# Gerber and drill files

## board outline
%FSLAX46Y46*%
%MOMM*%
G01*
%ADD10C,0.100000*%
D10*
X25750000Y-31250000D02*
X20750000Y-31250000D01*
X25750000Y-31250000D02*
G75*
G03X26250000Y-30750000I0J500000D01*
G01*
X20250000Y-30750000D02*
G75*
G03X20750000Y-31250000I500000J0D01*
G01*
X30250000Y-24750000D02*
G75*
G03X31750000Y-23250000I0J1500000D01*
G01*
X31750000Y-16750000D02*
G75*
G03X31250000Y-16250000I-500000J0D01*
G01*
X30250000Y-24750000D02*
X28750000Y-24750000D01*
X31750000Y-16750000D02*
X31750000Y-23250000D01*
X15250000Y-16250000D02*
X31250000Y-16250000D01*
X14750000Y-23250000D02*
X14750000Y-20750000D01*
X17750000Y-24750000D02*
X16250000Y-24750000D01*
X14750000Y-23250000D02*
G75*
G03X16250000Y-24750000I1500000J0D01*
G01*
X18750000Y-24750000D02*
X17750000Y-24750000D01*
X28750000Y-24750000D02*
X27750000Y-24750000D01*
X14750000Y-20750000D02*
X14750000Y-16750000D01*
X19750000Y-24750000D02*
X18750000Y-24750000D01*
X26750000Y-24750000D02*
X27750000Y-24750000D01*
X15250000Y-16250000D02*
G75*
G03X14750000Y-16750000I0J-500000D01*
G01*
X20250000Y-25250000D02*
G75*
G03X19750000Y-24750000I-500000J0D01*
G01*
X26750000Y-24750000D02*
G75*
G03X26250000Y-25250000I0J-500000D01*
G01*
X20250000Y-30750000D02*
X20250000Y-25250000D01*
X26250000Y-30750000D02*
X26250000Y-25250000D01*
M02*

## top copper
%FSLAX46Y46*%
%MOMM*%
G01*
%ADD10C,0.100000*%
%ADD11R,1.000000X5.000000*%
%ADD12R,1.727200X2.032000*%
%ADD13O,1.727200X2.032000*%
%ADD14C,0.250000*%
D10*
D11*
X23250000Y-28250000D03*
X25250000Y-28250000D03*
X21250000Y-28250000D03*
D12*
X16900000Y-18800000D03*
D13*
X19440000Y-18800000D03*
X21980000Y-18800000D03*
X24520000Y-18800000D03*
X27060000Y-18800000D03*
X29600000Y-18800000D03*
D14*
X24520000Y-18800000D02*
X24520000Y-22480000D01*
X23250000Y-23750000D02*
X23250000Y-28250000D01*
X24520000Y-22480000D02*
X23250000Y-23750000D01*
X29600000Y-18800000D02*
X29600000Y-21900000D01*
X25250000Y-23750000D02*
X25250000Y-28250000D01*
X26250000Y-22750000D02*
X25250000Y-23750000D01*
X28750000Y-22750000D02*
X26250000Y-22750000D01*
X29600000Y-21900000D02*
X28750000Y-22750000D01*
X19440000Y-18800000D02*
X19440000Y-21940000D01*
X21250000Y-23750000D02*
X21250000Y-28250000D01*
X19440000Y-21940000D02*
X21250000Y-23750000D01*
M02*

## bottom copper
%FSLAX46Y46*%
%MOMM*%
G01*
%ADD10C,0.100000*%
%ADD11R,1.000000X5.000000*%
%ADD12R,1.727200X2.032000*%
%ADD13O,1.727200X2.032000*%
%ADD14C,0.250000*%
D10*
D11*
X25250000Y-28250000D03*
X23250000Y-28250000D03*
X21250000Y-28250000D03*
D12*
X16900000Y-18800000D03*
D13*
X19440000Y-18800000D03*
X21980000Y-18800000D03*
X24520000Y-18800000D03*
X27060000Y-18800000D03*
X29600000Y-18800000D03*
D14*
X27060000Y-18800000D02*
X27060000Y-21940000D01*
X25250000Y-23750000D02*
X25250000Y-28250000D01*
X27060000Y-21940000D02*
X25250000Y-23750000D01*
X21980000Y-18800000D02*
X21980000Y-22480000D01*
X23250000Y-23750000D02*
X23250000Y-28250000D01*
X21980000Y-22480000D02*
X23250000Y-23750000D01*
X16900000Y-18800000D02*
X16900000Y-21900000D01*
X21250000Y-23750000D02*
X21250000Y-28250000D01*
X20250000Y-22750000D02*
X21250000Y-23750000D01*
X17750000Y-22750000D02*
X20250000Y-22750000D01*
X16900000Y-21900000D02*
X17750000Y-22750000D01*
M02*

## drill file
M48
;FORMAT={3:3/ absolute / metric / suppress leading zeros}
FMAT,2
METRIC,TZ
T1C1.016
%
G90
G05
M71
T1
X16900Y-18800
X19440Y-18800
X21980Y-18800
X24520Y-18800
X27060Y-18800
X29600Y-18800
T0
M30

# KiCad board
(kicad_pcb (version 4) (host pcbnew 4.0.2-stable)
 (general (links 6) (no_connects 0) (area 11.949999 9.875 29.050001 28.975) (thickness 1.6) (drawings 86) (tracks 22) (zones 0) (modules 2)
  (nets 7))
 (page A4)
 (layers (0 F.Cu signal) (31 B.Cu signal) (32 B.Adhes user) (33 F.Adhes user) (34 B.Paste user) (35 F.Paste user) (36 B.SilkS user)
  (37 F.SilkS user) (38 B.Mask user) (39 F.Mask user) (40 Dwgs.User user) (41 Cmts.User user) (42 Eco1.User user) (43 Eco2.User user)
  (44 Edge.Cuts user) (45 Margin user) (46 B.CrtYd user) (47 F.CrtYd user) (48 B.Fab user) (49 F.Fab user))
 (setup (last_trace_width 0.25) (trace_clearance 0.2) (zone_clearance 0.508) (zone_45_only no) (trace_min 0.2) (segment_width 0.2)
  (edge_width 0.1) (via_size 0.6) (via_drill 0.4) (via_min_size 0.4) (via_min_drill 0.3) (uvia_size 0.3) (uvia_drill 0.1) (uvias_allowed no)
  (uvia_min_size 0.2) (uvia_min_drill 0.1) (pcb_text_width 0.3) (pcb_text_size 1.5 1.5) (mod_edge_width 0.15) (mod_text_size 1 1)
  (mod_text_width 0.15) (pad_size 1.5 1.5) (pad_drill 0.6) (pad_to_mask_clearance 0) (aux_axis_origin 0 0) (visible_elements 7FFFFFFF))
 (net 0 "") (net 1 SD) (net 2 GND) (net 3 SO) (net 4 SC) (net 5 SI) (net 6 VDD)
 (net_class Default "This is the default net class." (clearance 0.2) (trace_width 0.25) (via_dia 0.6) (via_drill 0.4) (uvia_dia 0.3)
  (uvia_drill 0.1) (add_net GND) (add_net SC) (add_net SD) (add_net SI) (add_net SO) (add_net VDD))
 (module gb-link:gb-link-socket (layer F.Cu) (at 20.5 24)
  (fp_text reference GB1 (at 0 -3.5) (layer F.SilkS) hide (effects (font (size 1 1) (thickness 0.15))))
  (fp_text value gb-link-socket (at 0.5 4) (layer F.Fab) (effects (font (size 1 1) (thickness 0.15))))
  (pad 4 connect rect (at 0 0) (size 1 5) (layers F.Cu F.Mask) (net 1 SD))
  (pad 6 connect rect (at 2 0) (size 1 5) (layers F.Cu F.Mask) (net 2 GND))
  (pad 2 connect rect (at -2 0) (size 1 5) (layers F.Cu F.Mask) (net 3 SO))
  (pad 5 connect rect (at 2 0) (size 1 5) (layers B.Cu B.Mask) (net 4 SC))
  (pad 3 connect rect (at 0 0) (size 1 5) (layers B.Cu B.Mask) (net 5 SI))
  (pad 1 connect rect (at -2 0) (size 1 5) (layers B.Cu B.Mask) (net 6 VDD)))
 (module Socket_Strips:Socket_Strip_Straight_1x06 (layer F.Cu) (at 14.15 14.55)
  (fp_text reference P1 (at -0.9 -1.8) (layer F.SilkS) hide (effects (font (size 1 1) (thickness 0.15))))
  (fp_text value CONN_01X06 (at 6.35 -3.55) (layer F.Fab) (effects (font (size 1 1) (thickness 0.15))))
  (pad 1 thru_hole rect (at 0 0) (size 1.7272 2.032) (drill 1.016) (layers *.Cu *.Mask F.SilkS) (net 6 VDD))
  (pad 2 thru_hole oval (at 2.54 0) (size 1.7272 2.032) (drill 1.016) (layers *.Cu *.Mask F.SilkS) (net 3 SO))
  (pad 3 thru_hole oval (at 5.08 0) (size 1.7272 2.032) (drill 1.016) (layers *.Cu *.Mask F.SilkS) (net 5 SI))
  (pad 4 thru_hole oval (at 7.62 0) (size 1.7272 2.032) (drill 1.016) (layers *.Cu *.Mask F.SilkS) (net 1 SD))
  (pad 5 thru_hole oval (at 10.16 0) (size 1.7272 2.032) (drill 1.016) (layers *.Cu *.Mask F.SilkS) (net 4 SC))
  (pad 6 thru_hole oval (at 12.7 0) (size 1.7272 2.032) (drill 1.016) (layers *.Cu *.Mask F.SilkS) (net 2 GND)))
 (gr_line (start 23 27) (end 18 27) (angle 90) (layer Edge.Cuts) (width 0.1))
 (gr_arc (start 23 26.5) (end 23.5 26.5) (angle 90) (layer Edge.Cuts) (width 0.1))
 (gr_arc (start 18 26.5) (end 18 27) (angle 90) (layer Edge.Cuts) (width 0.1))
 (gr_arc (start 27.5 19) (end 29 19) (angle 90) (layer Edge.Cuts) (width 0.1))
 (gr_arc (start 28.5 12.5) (end 28.5 12) (angle 90) (layer Edge.Cuts) (width 0.1))
 (gr_line (start 27.5 20.5) (end 26 20.5) (angle 90) (layer Edge.Cuts) (width 0.1))
 (gr_line (start 29 12.5) (end 29 19) (angle 90) (layer Edge.Cuts) (width 0.1))
 (gr_line (start 12.5 12) (end 28.5 12) (angle 90) (layer Edge.Cuts) (width 0.1))
 (gr_line (start 12 19) (end 12 16.5) (angle 90) (layer Edge.Cuts) (width 0.1))
 (gr_line (start 15 20.5) (end 13.5 20.5) (angle 90) (layer Edge.Cuts) (width 0.1))
 (gr_arc (start 13.5 19) (end 13.5 20.5) (angle 90) (layer Edge.Cuts) (width 0.1))
 (gr_line (start 16 20.5) (end 15 20.5) (angle 90) (layer Edge.Cuts) (width 0.1))
 (gr_line (start 26 20.5) (end 25 20.5) (angle 90) (layer Edge.Cuts) (width 0.1))
 (gr_line (start 12 16.5) (end 12 12.5) (angle 90) (layer Edge.Cuts) (width 0.1))
 (gr_line (start 17 20.5) (end 16 20.5) (angle 90) (layer Edge.Cuts) (width 0.1))
 (gr_line (start 24 20.5) (end 25 20.5) (angle 90) (layer Edge.Cuts) (width 0.1))
 (gr_arc (start 12.5 12.5) (end 12 12.5) (angle 90) (layer Edge.Cuts) (width 0.1))
 (gr_arc (start 17 21) (end 17 20.5) (angle 90) (layer Edge.Cuts) (width 0.1))
 (gr_arc (start 24 21) (end 23.5 21) (angle 90) (layer Edge.Cuts) (width 0.1))
 (gr_line (start 17.5 26.5) (end 17.5 21) (angle 90) (layer Edge.Cuts) (width 0.1))
 (gr_line (start 23.5 26.5) (end 23.5 21) (angle 90) (layer Edge.Cuts) (width 0.1))
 (segment (start 21.77 14.55) (end 21.77 18.23) (width 0.25) (layer F.Cu) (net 1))
 (segment (start 20.5 19.5) (end 20.5 24) (width 0.25) (layer F.Cu) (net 1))
 (segment (start 21.77 18.23) (end 20.5 19.5) (width 0.25) (layer F.Cu) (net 1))
 (segment (start 26.85 14.55) (end 26.85 17.65) (width 0.25) (layer F.Cu) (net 2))
 (segment (start 22.5 19.5) (end 22.5 24) (width 0.25) (layer F.Cu) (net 2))
 (segment (start 23.5 18.5) (end 22.5 19.5) (width 0.25) (layer F.Cu) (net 2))
 (segment (start 26 18.5) (end 23.5 18.5) (width 0.25) (layer F.Cu) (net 2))
 (segment (start 26.85 17.65) (end 26 18.5) (width 0.25) (layer F.Cu) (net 2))
 (segment (start 16.69 14.55) (end 16.69 17.69) (width 0.25) (layer F.Cu) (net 3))
 (segment (start 18.5 19.5) (end 18.5 24) (width 0.25) (layer F.Cu) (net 3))
 (segment (start 16.69 17.69) (end 18.5 19.5) (width 0.25) (layer F.Cu) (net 3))
 (segment (start 24.31 14.55) (end 24.31 17.69) (width 0.25) (layer B.Cu) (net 4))
 (segment (start 22.5 19.5) (end 22.5 24) (width 0.25) (layer B.Cu) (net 4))
 (segment (start 24.31 17.69) (end 22.5 19.5) (width 0.25) (layer B.Cu) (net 4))
 (segment (start 19.23 14.55) (end 19.23 18.23) (width 0.25) (layer B.Cu) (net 5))
 (segment (start 20.5 19.5) (end 20.5 24) (width 0.25) (layer B.Cu) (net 5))
 (segment (start 19.23 18.23) (end 20.5 19.5) (width 0.25) (layer B.Cu) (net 5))
 (segment (start 14.15 14.55) (end 14.15 17.65) (width 0.25) (layer B.Cu) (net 6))
 (segment (start 18.5 19.5) (end 18.5 24) (width 0.25) (layer B.Cu) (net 6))
 (segment (start 17.5 18.5) (end 18.5 19.5) (width 0.25) (layer B.Cu) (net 6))
 (segment (start 15 18.5) (end 17.5 18.5) (width 0.25) (layer B.Cu) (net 6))
 (segment (start 14.15 17.65) (end 15 18.5) (width 0.25) (layer B.Cu) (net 6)))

